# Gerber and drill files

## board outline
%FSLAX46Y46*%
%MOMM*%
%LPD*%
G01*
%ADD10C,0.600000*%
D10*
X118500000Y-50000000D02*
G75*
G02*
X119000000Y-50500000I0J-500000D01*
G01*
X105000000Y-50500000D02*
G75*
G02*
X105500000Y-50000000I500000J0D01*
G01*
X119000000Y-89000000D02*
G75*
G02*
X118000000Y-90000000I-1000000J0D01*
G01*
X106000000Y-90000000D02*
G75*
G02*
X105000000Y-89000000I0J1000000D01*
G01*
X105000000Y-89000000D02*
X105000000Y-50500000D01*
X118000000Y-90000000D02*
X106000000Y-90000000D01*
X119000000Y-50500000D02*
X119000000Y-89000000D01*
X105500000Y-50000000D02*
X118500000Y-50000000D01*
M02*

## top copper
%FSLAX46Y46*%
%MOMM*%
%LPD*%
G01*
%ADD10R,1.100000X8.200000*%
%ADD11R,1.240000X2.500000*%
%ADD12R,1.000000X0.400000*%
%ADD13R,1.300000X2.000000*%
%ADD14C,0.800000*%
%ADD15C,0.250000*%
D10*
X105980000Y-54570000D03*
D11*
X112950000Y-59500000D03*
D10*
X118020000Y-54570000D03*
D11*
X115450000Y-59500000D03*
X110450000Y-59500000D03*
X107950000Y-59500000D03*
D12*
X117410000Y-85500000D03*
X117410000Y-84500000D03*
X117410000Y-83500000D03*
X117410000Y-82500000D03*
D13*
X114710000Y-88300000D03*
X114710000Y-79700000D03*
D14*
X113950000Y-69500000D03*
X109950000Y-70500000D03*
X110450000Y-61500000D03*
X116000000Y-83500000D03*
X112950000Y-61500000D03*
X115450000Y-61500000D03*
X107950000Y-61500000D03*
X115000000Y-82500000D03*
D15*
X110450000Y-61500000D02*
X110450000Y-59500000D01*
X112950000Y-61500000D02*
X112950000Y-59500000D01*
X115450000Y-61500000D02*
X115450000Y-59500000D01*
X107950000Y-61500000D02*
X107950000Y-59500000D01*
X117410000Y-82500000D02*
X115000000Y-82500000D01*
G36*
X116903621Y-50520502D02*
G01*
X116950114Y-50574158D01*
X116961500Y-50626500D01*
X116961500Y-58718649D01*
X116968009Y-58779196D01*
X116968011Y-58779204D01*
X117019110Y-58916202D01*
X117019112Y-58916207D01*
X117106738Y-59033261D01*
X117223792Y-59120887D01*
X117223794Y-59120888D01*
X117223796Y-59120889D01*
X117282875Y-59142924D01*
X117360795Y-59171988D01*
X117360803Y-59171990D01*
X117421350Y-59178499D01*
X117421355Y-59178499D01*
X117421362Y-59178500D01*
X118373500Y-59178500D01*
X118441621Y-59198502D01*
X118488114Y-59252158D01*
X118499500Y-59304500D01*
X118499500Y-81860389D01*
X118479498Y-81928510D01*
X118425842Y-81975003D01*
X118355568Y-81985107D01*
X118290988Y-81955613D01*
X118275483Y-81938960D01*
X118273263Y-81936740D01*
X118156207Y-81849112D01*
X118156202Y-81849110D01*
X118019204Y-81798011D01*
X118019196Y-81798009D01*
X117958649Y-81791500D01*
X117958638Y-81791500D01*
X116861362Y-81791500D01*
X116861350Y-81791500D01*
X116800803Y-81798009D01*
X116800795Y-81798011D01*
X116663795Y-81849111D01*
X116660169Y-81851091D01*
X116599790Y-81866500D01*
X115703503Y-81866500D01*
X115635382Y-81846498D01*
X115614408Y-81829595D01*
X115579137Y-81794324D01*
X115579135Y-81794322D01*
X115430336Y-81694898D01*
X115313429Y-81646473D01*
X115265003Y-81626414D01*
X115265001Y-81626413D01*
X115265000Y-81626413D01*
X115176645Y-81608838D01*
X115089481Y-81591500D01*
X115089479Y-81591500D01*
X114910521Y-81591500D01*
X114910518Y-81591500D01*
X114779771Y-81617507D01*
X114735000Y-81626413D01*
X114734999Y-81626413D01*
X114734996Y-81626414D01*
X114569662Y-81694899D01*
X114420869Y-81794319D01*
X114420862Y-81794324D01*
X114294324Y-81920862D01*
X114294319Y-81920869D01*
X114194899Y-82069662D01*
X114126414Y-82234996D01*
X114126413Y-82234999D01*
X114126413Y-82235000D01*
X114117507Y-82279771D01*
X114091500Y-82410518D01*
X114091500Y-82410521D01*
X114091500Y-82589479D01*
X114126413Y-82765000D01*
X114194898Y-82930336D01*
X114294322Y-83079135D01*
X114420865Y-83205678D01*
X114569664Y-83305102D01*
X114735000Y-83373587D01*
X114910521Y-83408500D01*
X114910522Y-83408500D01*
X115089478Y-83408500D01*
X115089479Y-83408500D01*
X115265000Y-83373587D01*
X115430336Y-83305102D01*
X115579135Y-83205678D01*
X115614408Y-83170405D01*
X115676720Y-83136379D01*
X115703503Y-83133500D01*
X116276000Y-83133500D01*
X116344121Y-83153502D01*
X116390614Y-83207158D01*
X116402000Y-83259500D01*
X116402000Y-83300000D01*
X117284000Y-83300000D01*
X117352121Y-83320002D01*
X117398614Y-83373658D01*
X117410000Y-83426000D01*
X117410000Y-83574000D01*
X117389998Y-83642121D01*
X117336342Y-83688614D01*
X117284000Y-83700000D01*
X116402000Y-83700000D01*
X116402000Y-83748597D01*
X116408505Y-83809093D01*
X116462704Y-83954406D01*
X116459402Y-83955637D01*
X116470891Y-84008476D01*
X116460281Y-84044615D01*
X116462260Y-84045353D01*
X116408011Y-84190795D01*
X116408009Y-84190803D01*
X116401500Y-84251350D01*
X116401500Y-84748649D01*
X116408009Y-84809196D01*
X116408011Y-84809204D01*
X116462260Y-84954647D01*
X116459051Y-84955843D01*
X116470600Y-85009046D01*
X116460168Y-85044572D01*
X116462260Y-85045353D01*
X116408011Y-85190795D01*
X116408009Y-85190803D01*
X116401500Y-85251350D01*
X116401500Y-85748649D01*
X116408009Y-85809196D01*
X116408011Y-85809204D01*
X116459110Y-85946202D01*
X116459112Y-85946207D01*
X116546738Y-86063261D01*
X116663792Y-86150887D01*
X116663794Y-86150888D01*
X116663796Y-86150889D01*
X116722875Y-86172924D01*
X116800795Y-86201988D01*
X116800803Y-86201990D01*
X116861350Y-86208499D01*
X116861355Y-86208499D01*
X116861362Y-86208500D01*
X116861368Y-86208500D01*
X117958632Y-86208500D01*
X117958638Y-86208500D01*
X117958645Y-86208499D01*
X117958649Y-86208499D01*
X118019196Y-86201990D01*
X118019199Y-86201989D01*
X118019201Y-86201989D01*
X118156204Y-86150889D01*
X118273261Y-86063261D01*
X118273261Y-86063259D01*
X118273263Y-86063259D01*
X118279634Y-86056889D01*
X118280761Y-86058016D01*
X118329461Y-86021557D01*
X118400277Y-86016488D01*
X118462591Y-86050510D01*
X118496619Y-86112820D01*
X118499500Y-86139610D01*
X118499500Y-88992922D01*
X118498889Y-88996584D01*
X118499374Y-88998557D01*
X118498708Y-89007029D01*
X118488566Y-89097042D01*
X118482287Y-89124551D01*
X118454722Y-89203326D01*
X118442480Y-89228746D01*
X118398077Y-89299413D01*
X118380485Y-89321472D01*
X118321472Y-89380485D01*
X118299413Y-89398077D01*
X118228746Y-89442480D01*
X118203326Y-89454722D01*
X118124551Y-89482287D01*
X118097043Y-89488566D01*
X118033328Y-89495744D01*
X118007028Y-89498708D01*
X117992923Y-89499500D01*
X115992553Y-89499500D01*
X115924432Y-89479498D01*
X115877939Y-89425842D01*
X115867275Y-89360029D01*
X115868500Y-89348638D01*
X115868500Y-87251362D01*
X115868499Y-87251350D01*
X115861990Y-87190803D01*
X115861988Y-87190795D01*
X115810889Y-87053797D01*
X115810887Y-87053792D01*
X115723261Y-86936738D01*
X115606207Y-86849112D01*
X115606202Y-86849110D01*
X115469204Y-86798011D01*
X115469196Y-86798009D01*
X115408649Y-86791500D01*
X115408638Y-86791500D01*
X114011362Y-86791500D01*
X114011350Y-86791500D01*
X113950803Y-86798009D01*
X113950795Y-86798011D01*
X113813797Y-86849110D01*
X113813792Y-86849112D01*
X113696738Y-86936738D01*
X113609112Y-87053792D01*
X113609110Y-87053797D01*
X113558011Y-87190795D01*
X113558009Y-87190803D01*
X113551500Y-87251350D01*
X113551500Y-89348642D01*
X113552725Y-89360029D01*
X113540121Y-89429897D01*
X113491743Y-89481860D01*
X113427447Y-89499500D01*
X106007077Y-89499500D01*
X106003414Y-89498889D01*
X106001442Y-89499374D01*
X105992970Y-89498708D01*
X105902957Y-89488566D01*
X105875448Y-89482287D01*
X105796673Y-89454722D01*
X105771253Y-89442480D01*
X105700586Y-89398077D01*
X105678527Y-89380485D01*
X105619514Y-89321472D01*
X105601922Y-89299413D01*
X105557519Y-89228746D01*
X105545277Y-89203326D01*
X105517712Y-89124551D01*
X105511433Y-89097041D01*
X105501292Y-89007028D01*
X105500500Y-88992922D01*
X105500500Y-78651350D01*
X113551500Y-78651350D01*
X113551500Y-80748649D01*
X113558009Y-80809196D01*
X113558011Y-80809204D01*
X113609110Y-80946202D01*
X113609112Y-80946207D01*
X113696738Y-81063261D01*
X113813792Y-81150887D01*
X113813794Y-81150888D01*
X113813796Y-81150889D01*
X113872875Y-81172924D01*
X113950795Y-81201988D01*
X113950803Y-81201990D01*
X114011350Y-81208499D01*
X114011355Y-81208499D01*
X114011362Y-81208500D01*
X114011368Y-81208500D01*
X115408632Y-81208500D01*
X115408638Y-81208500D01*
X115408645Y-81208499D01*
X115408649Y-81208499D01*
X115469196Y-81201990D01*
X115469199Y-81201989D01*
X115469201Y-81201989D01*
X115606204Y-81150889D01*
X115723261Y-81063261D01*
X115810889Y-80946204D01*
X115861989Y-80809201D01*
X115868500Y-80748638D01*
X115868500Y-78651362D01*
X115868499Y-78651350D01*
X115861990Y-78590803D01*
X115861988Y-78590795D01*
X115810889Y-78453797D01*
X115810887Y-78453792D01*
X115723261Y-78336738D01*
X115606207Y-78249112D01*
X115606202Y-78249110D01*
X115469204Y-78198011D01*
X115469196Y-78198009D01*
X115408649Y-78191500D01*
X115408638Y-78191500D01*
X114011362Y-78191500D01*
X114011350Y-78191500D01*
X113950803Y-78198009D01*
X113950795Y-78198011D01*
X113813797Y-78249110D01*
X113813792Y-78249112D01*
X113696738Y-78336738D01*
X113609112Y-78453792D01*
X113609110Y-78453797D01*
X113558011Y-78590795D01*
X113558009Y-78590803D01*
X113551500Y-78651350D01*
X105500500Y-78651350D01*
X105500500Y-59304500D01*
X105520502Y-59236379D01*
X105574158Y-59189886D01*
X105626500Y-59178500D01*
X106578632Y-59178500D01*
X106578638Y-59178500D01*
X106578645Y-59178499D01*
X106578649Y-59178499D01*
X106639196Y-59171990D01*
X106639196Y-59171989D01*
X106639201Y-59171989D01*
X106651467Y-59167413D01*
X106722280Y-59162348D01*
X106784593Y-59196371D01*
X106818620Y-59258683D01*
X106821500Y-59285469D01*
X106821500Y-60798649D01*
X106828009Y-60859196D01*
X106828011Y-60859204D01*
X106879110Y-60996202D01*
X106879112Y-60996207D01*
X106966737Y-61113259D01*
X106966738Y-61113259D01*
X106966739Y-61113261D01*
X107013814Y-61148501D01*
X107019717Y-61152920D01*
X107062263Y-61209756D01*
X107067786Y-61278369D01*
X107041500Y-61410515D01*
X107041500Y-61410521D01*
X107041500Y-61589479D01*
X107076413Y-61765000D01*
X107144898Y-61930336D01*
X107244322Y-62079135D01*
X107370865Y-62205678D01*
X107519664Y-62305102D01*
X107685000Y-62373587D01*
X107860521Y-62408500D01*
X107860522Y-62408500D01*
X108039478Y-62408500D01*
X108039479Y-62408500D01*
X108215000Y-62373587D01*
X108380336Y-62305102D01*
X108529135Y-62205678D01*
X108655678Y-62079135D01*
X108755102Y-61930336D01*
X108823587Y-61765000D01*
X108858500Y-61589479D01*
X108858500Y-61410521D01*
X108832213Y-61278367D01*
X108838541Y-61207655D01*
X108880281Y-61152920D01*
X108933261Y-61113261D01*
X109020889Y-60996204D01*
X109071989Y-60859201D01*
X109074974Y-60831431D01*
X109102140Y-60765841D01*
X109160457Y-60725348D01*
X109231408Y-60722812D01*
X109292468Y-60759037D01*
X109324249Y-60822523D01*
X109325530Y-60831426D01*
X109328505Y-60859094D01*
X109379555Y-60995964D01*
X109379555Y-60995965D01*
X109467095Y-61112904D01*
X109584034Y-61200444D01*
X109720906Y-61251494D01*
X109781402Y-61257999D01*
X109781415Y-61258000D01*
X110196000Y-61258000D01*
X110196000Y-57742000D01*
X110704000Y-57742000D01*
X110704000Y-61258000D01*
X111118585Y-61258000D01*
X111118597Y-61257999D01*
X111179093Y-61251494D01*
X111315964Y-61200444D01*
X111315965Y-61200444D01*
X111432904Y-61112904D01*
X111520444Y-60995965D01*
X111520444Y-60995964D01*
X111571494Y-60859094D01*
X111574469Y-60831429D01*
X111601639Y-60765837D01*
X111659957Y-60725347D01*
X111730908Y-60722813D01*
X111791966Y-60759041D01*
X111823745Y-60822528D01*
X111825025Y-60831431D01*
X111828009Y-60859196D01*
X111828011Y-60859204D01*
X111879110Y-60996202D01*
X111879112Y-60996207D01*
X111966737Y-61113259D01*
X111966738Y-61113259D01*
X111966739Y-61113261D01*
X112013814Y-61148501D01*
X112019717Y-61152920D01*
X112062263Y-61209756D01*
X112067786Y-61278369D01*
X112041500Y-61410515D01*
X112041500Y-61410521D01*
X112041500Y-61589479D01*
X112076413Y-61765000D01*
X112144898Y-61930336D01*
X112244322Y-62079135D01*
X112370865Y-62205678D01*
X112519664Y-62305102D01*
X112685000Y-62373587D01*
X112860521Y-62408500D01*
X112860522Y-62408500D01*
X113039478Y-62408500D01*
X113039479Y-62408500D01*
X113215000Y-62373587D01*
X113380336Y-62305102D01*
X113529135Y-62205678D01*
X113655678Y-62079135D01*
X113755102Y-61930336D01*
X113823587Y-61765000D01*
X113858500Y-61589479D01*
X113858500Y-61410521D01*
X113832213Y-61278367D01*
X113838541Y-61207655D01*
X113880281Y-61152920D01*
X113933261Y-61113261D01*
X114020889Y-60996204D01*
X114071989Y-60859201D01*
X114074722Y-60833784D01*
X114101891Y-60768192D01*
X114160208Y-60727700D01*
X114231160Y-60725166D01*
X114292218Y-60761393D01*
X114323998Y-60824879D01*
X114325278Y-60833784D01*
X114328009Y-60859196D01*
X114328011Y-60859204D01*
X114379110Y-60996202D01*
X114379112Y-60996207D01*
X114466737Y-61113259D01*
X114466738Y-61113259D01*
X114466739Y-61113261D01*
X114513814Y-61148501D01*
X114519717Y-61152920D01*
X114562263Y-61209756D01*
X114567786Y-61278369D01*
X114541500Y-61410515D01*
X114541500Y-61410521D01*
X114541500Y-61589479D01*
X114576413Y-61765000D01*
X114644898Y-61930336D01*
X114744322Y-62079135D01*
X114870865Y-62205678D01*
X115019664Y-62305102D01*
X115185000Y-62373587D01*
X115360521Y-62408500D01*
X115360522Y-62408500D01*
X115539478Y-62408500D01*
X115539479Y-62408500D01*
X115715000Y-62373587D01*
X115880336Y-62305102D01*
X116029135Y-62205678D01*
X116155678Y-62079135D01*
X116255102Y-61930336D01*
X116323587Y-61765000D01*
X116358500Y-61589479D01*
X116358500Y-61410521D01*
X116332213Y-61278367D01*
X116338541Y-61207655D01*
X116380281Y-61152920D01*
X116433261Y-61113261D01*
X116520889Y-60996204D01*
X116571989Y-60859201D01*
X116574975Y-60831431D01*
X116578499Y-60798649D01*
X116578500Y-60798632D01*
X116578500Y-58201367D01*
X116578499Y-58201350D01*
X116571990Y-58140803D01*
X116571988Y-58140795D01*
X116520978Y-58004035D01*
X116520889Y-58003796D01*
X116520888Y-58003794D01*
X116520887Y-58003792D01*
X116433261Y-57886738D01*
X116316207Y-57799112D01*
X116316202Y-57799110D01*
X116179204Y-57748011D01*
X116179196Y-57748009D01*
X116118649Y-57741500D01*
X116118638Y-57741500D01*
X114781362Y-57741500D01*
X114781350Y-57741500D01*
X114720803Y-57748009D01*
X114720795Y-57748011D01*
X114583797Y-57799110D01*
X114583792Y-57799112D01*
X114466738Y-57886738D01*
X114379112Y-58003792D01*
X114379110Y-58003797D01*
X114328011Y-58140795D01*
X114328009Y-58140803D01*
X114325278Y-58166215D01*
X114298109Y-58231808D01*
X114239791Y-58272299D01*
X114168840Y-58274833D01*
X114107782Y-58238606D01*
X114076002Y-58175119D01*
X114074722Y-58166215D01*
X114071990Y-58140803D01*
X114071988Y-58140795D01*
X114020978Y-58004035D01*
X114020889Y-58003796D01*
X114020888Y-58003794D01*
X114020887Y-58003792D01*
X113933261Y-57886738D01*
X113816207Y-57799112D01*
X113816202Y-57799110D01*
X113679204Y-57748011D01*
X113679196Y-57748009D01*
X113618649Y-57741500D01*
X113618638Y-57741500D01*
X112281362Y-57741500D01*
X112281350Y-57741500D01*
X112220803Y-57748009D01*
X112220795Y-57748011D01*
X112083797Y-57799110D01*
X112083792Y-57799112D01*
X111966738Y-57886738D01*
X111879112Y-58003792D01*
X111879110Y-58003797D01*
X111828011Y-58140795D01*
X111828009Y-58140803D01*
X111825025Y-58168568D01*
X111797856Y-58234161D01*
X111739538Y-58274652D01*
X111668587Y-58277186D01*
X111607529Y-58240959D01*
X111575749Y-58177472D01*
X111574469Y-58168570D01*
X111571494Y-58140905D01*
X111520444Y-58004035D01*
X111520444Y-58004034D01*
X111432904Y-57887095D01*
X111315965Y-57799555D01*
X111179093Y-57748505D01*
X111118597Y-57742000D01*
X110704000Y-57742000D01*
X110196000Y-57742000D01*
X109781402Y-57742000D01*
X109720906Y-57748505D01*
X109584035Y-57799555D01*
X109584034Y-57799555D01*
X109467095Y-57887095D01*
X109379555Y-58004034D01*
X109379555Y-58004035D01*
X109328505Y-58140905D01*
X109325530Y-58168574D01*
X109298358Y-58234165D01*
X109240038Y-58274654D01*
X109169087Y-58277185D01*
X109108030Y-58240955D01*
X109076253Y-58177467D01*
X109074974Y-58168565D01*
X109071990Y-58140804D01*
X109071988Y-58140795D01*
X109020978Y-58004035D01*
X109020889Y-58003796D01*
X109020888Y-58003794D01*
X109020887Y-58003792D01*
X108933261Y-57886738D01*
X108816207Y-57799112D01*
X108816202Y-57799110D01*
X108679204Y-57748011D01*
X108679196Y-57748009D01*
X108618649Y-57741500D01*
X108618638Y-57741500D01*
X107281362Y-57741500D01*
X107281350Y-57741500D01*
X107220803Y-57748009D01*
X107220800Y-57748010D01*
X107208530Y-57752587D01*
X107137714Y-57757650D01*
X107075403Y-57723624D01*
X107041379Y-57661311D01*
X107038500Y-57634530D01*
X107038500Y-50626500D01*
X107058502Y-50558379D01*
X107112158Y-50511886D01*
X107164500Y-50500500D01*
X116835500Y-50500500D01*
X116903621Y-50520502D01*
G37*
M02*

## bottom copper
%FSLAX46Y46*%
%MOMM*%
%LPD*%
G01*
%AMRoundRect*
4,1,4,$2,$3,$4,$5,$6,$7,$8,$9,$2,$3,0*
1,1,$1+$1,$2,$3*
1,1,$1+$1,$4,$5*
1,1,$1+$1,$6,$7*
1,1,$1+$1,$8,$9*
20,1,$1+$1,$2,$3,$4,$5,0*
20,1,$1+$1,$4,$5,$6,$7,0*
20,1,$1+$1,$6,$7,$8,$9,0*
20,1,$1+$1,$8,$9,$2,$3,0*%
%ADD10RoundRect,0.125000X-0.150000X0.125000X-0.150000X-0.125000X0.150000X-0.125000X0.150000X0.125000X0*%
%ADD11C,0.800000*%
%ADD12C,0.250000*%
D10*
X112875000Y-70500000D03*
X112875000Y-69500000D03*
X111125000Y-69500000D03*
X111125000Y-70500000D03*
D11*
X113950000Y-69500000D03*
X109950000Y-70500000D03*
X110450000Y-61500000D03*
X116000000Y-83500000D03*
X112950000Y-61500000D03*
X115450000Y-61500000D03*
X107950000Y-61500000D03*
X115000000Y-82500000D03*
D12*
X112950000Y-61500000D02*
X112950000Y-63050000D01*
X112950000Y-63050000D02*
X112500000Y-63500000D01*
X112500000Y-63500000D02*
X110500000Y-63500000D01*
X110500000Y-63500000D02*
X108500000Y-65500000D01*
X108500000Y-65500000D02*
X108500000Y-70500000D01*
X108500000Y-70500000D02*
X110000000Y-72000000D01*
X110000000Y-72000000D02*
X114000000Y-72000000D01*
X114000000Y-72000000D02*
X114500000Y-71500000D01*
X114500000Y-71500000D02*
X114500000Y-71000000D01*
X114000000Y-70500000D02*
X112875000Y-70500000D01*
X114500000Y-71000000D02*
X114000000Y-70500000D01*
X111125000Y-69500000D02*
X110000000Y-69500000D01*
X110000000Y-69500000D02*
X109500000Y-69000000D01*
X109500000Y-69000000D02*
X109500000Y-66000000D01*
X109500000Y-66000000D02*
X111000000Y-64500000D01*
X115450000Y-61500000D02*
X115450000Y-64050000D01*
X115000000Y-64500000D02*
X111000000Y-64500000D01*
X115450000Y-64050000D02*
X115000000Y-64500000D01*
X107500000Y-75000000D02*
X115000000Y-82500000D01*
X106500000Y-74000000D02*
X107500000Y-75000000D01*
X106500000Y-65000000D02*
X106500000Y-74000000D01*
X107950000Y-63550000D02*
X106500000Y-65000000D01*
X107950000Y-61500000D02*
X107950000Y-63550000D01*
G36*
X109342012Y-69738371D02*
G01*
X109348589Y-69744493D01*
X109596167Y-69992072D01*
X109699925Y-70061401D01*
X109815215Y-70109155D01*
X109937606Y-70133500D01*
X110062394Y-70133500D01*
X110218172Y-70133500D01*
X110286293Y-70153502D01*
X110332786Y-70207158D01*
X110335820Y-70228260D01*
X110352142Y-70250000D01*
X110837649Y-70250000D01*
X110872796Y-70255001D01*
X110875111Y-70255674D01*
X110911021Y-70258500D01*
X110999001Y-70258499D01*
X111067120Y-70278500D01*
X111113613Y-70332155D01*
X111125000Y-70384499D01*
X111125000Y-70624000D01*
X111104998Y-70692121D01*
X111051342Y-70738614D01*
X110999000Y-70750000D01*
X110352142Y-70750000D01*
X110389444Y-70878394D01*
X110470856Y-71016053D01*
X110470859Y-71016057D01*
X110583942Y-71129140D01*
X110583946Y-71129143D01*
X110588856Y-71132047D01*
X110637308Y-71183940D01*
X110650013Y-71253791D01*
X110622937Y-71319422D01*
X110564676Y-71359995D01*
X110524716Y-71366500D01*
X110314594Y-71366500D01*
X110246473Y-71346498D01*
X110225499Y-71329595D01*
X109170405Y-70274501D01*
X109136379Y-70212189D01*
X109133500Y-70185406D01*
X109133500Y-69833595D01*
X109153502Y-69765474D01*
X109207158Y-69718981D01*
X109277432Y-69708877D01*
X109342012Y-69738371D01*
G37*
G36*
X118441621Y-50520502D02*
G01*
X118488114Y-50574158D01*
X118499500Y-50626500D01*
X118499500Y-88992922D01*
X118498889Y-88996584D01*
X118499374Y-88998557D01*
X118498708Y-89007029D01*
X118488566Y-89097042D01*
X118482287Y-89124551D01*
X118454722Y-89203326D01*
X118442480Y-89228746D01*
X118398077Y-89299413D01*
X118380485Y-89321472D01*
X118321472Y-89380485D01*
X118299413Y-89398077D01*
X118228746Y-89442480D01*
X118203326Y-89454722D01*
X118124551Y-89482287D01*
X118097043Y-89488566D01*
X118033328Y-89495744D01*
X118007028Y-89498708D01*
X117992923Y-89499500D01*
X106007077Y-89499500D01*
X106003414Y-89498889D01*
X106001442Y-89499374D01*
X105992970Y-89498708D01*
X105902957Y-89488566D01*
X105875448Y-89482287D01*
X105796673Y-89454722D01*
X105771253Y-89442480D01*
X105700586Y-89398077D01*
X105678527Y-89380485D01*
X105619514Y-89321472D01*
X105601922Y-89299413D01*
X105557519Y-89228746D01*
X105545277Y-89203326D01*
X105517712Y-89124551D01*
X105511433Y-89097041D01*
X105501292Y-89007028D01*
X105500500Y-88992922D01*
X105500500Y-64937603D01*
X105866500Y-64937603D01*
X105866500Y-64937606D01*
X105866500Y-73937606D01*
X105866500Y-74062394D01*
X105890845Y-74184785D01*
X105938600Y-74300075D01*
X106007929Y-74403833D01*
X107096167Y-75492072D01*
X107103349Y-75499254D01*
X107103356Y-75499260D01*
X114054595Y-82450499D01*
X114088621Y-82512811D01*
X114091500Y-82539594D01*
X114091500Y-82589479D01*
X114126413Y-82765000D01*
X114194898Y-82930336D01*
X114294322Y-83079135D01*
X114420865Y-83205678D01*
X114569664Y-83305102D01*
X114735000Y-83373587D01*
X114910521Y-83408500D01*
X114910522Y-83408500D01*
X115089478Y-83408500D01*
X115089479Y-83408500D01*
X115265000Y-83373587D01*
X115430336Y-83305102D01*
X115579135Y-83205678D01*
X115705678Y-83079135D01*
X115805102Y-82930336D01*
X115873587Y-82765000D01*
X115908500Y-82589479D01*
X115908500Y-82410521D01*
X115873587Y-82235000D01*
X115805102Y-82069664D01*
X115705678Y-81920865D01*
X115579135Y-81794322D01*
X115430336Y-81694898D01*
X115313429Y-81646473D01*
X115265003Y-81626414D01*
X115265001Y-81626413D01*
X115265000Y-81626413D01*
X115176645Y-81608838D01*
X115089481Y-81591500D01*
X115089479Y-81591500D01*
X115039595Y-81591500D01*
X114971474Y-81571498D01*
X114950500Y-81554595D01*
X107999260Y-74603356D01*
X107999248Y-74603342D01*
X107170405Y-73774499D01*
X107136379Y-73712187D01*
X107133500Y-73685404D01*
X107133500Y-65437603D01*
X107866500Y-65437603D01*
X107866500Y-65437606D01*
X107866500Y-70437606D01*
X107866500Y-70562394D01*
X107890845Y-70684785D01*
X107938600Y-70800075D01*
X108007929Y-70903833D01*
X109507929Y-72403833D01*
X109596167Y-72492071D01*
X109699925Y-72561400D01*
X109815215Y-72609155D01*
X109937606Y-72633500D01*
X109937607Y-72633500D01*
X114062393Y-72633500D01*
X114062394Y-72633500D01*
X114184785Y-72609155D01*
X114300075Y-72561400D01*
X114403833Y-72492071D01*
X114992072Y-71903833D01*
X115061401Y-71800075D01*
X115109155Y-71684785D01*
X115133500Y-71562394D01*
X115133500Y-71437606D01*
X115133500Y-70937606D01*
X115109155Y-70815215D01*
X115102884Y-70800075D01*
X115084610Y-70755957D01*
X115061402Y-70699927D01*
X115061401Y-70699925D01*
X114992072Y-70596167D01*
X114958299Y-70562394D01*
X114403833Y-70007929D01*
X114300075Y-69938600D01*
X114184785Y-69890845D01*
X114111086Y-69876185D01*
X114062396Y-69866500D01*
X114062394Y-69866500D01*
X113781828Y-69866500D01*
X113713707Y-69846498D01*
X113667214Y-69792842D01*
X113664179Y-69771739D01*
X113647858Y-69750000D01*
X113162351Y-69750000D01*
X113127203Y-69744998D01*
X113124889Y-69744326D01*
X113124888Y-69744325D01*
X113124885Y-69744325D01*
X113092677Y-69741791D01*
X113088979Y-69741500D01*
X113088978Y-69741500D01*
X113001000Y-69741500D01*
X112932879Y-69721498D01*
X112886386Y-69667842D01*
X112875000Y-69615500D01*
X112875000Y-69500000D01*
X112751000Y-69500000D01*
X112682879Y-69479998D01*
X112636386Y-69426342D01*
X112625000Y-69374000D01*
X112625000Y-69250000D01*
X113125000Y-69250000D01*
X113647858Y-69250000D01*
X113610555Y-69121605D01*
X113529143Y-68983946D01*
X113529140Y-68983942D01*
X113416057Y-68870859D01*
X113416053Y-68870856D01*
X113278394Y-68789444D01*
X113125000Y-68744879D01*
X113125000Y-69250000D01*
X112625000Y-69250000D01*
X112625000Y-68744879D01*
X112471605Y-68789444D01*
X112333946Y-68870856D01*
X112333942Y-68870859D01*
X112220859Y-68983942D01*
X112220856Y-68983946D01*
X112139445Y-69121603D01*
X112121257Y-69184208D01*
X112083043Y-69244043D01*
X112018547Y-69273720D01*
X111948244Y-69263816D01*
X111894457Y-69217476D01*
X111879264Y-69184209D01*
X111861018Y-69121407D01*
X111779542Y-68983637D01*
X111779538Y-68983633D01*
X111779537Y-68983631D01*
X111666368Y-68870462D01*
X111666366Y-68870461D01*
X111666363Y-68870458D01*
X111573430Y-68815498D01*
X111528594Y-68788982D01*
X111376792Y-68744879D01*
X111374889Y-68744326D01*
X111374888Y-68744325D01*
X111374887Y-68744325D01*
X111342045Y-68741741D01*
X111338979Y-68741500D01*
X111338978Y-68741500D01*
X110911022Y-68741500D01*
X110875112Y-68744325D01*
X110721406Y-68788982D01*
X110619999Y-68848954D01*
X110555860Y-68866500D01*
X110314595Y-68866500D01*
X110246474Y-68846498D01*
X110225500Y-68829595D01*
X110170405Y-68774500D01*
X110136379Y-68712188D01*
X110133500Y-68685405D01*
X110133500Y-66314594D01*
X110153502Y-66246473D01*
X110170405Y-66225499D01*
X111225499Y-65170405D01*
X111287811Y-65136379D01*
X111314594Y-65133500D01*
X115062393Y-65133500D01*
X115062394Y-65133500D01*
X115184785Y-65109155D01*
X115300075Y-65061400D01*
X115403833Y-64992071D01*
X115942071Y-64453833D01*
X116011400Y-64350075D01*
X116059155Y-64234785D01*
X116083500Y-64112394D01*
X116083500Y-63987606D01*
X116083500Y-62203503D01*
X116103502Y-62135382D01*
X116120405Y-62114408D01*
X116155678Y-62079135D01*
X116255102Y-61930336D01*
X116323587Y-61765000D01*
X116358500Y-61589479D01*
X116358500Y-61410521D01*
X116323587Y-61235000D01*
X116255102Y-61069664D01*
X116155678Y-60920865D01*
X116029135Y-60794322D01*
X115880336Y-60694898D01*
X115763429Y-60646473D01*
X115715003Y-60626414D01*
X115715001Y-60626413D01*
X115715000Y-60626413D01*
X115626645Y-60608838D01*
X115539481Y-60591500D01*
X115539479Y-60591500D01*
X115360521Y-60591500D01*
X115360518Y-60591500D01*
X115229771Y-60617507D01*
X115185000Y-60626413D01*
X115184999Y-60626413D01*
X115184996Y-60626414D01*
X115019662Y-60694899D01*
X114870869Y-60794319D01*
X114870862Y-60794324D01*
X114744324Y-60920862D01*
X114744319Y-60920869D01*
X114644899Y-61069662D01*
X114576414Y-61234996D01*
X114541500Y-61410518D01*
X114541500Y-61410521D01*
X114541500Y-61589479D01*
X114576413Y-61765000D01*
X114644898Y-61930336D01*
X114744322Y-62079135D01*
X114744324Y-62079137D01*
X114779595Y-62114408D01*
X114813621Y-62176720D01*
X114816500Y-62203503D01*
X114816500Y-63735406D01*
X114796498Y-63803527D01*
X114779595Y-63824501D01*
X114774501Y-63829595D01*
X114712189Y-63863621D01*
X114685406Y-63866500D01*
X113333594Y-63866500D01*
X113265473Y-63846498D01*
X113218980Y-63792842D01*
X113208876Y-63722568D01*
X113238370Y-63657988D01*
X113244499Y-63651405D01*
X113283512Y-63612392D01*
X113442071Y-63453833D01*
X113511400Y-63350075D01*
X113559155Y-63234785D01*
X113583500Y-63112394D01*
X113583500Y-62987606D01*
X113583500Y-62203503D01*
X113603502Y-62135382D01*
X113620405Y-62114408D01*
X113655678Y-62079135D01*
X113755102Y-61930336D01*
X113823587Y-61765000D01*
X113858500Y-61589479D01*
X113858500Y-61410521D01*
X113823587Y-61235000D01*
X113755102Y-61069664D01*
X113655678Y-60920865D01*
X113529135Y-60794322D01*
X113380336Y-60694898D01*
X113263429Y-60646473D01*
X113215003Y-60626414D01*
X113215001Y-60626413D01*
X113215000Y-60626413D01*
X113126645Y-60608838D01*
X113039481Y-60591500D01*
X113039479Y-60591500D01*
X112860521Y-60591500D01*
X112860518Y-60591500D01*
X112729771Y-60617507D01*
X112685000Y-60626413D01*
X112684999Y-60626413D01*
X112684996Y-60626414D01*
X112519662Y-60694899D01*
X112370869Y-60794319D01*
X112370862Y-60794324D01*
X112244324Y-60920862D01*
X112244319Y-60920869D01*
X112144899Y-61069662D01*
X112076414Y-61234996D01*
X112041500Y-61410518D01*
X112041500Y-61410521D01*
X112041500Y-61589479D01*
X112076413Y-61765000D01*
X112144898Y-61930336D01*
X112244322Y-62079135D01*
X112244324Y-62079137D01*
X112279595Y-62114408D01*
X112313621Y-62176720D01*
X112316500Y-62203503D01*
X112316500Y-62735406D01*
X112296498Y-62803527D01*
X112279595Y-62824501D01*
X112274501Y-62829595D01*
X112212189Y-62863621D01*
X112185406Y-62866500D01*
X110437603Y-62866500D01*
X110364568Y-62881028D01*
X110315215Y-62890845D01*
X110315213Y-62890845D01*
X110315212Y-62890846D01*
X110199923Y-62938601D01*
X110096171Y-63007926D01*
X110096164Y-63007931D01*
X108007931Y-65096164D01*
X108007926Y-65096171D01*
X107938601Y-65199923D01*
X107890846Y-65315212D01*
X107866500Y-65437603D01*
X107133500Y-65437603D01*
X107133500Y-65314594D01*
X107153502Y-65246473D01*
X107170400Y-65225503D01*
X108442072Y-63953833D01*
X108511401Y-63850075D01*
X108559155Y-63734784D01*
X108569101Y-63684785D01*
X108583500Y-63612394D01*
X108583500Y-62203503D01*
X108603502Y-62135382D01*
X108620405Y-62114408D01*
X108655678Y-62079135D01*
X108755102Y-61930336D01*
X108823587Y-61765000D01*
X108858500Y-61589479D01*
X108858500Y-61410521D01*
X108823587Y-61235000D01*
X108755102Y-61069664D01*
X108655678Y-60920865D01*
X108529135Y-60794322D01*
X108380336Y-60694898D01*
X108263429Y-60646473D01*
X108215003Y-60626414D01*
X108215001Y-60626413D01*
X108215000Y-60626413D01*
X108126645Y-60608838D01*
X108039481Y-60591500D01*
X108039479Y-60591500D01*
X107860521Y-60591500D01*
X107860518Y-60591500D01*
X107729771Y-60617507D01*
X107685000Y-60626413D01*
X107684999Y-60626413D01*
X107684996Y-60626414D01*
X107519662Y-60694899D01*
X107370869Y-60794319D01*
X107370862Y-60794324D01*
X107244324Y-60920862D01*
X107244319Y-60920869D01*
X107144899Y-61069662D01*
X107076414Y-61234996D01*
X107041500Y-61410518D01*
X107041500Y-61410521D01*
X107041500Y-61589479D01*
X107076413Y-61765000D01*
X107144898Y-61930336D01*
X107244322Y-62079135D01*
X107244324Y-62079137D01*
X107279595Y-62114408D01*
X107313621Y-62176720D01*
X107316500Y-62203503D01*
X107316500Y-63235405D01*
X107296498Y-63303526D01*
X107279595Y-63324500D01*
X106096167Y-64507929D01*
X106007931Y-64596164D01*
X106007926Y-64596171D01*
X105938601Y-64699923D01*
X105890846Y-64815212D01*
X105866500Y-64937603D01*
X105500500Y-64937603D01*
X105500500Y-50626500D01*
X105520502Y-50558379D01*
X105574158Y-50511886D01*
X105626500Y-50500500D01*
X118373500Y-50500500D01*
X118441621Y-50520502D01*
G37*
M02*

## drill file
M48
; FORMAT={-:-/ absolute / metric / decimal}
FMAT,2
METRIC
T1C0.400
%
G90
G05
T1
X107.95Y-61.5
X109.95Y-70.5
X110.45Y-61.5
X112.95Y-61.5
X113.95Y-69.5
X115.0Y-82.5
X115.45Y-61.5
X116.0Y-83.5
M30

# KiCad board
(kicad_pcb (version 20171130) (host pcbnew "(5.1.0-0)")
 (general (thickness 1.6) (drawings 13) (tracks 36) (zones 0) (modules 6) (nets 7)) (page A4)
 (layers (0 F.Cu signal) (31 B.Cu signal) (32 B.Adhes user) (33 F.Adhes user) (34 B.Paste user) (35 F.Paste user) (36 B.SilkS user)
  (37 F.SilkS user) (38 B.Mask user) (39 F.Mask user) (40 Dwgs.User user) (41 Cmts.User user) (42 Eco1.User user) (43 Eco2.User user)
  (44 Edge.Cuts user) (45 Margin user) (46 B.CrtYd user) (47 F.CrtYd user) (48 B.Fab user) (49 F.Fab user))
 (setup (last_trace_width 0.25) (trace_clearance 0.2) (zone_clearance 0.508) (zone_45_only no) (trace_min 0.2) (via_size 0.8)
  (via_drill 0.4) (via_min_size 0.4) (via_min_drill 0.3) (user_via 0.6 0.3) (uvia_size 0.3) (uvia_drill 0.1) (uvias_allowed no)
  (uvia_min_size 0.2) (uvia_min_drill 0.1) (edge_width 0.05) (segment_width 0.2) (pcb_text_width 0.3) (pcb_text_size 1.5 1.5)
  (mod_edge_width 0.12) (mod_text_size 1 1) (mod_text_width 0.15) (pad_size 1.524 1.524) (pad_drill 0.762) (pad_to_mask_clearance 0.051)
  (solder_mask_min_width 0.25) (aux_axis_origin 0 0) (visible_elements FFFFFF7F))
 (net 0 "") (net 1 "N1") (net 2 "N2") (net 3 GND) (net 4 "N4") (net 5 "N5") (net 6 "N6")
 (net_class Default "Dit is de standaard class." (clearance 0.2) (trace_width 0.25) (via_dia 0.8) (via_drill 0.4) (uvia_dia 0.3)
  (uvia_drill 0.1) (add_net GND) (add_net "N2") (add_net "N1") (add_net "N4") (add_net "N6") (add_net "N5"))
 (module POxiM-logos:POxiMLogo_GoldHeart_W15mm (layer F.Cu) (at 114.5 69.5 90)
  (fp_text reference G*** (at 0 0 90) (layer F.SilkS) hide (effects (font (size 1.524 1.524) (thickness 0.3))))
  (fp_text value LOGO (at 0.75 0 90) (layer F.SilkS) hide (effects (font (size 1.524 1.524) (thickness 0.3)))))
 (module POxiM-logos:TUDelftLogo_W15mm (layer F.Cu) (at 108.5 69.5 90)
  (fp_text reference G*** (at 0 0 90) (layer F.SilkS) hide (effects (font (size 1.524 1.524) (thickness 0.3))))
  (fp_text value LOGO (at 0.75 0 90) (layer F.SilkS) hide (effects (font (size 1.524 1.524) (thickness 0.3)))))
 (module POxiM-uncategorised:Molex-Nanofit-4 (layer F.Cu) (at 112 59.5)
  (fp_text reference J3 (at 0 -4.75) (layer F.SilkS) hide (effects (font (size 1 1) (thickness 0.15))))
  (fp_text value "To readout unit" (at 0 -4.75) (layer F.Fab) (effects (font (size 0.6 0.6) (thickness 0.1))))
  (pad "" smd rect (at -6.02 -4.93) (size 1.1 8.2) (layers F.Cu F.Paste F.Mask))
  (pad 3 smd rect (at 0.95 0) (size 1.24 2.5) (layers F.Cu F.Paste F.Mask) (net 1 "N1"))
  (pad "" smd rect (at 6.02 -4.93) (size 1.1 8.2) (layers F.Cu F.Paste F.Mask))
  (pad 4 smd rect (at 3.45 0) (size 1.24 2.5) (layers F.Cu F.Paste F.Mask) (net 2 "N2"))
  (pad 2 smd rect (at -1.55 0) (size 1.24 2.5) (layers F.Cu F.Paste F.Mask) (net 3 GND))
  (pad 1 smd rect (at -4.05 0) (size 1.24 2.5) (layers F.Cu F.Paste F.Mask) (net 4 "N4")))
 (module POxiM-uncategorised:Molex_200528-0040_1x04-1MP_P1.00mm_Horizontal (layer F.Cu) (at 116.5 84 270)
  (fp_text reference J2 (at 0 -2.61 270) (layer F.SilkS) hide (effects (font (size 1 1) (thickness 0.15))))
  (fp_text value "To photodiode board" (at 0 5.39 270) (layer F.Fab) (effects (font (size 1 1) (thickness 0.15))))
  (pad 4 smd rect (at 1.5 -0.91 270) (size 0.4 1) (layers F.Cu F.Paste F.Mask) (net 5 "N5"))
  (pad 3 smd rect (at 0.5 -0.91 270) (size 0.4 1) (layers F.Cu F.Paste F.Mask) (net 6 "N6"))
  (pad 2 smd rect (at -0.5 -0.91 270) (size 0.4 1) (layers F.Cu F.Paste F.Mask) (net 3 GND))
  (pad 1 smd rect (at -1.5 -0.91 270) (size 0.4 1) (layers F.Cu F.Paste F.Mask) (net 4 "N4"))
  (pad MP smd rect (at 4.3 1.79 270) (size 2 1.3) (layers F.Cu F.Paste F.Mask))
  (pad MP smd rect (at -4.3 1.79 270) (size 2 1.3) (layers F.Cu F.Paste F.Mask)))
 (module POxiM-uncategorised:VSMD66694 (layer B.Cu) (at 112 70)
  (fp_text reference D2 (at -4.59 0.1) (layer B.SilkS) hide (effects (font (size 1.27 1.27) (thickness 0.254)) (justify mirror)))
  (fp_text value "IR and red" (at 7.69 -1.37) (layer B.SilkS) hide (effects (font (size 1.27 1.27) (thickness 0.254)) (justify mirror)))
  (pad 4 smd roundrect (at 0.875 0.5 270) (size 0.5 0.55) (layers B.Cu B.Paste B.Mask) (roundrect_rratio 0.25) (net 1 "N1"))
  (pad 3 smd roundrect (at 0.875 -0.5 270) (size 0.5 0.55) (layers B.Cu B.Paste B.Mask) (roundrect_rratio 0.25) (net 3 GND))
  (pad 2 smd roundrect (at -0.875 -0.5 270) (size 0.5 0.55) (layers B.Cu B.Paste B.Mask) (roundrect_rratio 0.25) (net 2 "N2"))
  (pad 1 smd roundrect (at -0.875 0.5 270) (size 0.5 0.55) (layers B.Cu B.Paste B.Mask) (roundrect_rratio 0.25) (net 3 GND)))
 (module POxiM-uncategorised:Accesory (layer F.Cu) (at 40 145)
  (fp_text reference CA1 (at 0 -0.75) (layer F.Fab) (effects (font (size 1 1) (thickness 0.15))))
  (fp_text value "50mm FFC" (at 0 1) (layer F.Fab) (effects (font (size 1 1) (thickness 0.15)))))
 (gr_arc (start 118.5 50.5) (end 119 50.5) (angle -90) (layer Edge.Cuts) (width 0.6))
 (gr_arc (start 105.5 50.5) (end 105.5 50) (angle -90) (layer Edge.Cuts) (width 0.6))
 (gr_arc (start 118 89) (end 118 90) (angle -90) (layer Edge.Cuts) (width 0.6))
 (gr_arc (start 106 89) (end 105 89) (angle -90) (layer Edge.Cuts) (width 0.6))
 (gr_line (start 105 89) (end 105 50.5) (layer Edge.Cuts) (width 0.6))
 (gr_line (start 118 90) (end 106 90) (layer Edge.Cuts) (width 0.6))
 (gr_line (start 119 50.5) (end 119 89) (layer Edge.Cuts) (width 0.6))
 (gr_line (start 105.5 50) (end 118.5 50) (layer Edge.Cuts) (width 0.6))
 (via (at 113.95 69.5) (size 0.8) (drill 0.4) (layers F.Cu B.Cu) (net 3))
 (via (at 109.95 70.5) (size 0.8) (drill 0.4) (layers F.Cu B.Cu) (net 3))
 (via (at 110.45 61.5) (size 0.8) (drill 0.4) (layers F.Cu B.Cu) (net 3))
 (segment (start 110.45 61.5) (end 110.45 59.5) (width 0.25) (layer F.Cu) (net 3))
 (via (at 116 83.5) (size 0.8) (drill 0.4) (layers F.Cu B.Cu) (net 3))
 (via (at 112.95 61.5) (size 0.8) (drill 0.4) (layers F.Cu B.Cu) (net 1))
 (segment (start 112.95 61.5) (end 112.95 59.5) (width 0.25) (layer F.Cu) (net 1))
 (segment (start 112.95 61.5) (end 112.95 63.05) (width 0.25) (layer B.Cu) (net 1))
 (segment (start 112.95 63.05) (end 112.5 63.5) (width 0.25) (layer B.Cu) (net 1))
 (segment (start 112.5 63.5) (end 110.5 63.5) (width 0.25) (layer B.Cu) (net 1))
 (segment (start 110.5 63.5) (end 108.5 65.5) (width 0.25) (layer B.Cu) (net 1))
 (segment (start 108.5 65.5) (end 108.5 70.5) (width 0.25) (layer B.Cu) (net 1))
 (segment (start 108.5 70.5) (end 110 72) (width 0.25) (layer B.Cu) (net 1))
 (segment (start 110 72) (end 114 72) (width 0.25) (layer B.Cu) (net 1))
 (segment (start 114 72) (end 114.5 71.5) (width 0.25) (layer B.Cu) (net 1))
 (segment (start 114.5 71.5) (end 114.5 71) (width 0.25) (layer B.Cu) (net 1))
 (segment (start 114 70.5) (end 112.875 70.5) (width 0.25) (layer B.Cu) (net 1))
 (segment (start 114.5 71) (end 114 70.5) (width 0.25) (layer B.Cu) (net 1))
 (segment (start 111.125 69.5) (end 110 69.5) (width 0.25) (layer B.Cu) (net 2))
 (segment (start 110 69.5) (end 109.5 69) (width 0.25) (layer B.Cu) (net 2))
 (segment (start 109.5 69) (end 109.5 66) (width 0.25) (layer B.Cu) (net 2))
 (segment (start 109.5 66) (end 111 64.5) (width 0.25) (layer B.Cu) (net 2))
 (via (at 115.45 61.5) (size 0.8) (drill 0.4) (layers F.Cu B.Cu) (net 2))
 (segment (start 115.45 61.5) (end 115.45 59.5) (width 0.25) (layer F.Cu) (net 2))
 (segment (start 115.45 61.5) (end 115.45 64.05) (width 0.25) (layer B.Cu) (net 2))
 (segment (start 115 64.5) (end 111 64.5) (width 0.25) (layer B.Cu) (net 2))
 (segment (start 115.45 64.05) (end 115 64.5) (width 0.25) (layer B.Cu) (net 2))
 (via (at 107.95 61.5) (size 0.8) (drill 0.4) (layers F.Cu B.Cu) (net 4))
 (segment (start 107.95 61.5) (end 107.95 59.5) (width 0.25) (layer F.Cu) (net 4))
 (segment (start 117.41 82.5) (end 115 82.5) (width 0.25) (layer F.Cu) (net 4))
 (via (at 115 82.5) (size 0.8) (drill 0.4) (layers F.Cu B.Cu) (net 4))
 (segment (start 107.5 75) (end 115 82.5) (width 0.25) (layer B.Cu) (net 4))
 (segment (start 106.5 74) (end 107.5 75) (width 0.25) (layer B.Cu) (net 4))
 (segment (start 106.5 65) (end 106.5 74) (width 0.25) (layer B.Cu) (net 4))
 (segment (start 107.95 63.55) (end 106.5 65) (width 0.25) (layer B.Cu) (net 4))
 (segment (start 107.95 61.5) (end 107.95 63.55) (width 0.25) (layer B.Cu) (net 4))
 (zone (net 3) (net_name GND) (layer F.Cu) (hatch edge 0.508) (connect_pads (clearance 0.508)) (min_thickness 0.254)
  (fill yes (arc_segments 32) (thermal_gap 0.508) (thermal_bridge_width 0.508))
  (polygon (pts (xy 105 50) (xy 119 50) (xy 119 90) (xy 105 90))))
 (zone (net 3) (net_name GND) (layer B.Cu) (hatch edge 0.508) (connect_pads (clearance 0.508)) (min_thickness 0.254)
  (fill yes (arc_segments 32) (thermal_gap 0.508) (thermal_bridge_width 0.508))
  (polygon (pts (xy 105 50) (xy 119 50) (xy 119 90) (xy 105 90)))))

